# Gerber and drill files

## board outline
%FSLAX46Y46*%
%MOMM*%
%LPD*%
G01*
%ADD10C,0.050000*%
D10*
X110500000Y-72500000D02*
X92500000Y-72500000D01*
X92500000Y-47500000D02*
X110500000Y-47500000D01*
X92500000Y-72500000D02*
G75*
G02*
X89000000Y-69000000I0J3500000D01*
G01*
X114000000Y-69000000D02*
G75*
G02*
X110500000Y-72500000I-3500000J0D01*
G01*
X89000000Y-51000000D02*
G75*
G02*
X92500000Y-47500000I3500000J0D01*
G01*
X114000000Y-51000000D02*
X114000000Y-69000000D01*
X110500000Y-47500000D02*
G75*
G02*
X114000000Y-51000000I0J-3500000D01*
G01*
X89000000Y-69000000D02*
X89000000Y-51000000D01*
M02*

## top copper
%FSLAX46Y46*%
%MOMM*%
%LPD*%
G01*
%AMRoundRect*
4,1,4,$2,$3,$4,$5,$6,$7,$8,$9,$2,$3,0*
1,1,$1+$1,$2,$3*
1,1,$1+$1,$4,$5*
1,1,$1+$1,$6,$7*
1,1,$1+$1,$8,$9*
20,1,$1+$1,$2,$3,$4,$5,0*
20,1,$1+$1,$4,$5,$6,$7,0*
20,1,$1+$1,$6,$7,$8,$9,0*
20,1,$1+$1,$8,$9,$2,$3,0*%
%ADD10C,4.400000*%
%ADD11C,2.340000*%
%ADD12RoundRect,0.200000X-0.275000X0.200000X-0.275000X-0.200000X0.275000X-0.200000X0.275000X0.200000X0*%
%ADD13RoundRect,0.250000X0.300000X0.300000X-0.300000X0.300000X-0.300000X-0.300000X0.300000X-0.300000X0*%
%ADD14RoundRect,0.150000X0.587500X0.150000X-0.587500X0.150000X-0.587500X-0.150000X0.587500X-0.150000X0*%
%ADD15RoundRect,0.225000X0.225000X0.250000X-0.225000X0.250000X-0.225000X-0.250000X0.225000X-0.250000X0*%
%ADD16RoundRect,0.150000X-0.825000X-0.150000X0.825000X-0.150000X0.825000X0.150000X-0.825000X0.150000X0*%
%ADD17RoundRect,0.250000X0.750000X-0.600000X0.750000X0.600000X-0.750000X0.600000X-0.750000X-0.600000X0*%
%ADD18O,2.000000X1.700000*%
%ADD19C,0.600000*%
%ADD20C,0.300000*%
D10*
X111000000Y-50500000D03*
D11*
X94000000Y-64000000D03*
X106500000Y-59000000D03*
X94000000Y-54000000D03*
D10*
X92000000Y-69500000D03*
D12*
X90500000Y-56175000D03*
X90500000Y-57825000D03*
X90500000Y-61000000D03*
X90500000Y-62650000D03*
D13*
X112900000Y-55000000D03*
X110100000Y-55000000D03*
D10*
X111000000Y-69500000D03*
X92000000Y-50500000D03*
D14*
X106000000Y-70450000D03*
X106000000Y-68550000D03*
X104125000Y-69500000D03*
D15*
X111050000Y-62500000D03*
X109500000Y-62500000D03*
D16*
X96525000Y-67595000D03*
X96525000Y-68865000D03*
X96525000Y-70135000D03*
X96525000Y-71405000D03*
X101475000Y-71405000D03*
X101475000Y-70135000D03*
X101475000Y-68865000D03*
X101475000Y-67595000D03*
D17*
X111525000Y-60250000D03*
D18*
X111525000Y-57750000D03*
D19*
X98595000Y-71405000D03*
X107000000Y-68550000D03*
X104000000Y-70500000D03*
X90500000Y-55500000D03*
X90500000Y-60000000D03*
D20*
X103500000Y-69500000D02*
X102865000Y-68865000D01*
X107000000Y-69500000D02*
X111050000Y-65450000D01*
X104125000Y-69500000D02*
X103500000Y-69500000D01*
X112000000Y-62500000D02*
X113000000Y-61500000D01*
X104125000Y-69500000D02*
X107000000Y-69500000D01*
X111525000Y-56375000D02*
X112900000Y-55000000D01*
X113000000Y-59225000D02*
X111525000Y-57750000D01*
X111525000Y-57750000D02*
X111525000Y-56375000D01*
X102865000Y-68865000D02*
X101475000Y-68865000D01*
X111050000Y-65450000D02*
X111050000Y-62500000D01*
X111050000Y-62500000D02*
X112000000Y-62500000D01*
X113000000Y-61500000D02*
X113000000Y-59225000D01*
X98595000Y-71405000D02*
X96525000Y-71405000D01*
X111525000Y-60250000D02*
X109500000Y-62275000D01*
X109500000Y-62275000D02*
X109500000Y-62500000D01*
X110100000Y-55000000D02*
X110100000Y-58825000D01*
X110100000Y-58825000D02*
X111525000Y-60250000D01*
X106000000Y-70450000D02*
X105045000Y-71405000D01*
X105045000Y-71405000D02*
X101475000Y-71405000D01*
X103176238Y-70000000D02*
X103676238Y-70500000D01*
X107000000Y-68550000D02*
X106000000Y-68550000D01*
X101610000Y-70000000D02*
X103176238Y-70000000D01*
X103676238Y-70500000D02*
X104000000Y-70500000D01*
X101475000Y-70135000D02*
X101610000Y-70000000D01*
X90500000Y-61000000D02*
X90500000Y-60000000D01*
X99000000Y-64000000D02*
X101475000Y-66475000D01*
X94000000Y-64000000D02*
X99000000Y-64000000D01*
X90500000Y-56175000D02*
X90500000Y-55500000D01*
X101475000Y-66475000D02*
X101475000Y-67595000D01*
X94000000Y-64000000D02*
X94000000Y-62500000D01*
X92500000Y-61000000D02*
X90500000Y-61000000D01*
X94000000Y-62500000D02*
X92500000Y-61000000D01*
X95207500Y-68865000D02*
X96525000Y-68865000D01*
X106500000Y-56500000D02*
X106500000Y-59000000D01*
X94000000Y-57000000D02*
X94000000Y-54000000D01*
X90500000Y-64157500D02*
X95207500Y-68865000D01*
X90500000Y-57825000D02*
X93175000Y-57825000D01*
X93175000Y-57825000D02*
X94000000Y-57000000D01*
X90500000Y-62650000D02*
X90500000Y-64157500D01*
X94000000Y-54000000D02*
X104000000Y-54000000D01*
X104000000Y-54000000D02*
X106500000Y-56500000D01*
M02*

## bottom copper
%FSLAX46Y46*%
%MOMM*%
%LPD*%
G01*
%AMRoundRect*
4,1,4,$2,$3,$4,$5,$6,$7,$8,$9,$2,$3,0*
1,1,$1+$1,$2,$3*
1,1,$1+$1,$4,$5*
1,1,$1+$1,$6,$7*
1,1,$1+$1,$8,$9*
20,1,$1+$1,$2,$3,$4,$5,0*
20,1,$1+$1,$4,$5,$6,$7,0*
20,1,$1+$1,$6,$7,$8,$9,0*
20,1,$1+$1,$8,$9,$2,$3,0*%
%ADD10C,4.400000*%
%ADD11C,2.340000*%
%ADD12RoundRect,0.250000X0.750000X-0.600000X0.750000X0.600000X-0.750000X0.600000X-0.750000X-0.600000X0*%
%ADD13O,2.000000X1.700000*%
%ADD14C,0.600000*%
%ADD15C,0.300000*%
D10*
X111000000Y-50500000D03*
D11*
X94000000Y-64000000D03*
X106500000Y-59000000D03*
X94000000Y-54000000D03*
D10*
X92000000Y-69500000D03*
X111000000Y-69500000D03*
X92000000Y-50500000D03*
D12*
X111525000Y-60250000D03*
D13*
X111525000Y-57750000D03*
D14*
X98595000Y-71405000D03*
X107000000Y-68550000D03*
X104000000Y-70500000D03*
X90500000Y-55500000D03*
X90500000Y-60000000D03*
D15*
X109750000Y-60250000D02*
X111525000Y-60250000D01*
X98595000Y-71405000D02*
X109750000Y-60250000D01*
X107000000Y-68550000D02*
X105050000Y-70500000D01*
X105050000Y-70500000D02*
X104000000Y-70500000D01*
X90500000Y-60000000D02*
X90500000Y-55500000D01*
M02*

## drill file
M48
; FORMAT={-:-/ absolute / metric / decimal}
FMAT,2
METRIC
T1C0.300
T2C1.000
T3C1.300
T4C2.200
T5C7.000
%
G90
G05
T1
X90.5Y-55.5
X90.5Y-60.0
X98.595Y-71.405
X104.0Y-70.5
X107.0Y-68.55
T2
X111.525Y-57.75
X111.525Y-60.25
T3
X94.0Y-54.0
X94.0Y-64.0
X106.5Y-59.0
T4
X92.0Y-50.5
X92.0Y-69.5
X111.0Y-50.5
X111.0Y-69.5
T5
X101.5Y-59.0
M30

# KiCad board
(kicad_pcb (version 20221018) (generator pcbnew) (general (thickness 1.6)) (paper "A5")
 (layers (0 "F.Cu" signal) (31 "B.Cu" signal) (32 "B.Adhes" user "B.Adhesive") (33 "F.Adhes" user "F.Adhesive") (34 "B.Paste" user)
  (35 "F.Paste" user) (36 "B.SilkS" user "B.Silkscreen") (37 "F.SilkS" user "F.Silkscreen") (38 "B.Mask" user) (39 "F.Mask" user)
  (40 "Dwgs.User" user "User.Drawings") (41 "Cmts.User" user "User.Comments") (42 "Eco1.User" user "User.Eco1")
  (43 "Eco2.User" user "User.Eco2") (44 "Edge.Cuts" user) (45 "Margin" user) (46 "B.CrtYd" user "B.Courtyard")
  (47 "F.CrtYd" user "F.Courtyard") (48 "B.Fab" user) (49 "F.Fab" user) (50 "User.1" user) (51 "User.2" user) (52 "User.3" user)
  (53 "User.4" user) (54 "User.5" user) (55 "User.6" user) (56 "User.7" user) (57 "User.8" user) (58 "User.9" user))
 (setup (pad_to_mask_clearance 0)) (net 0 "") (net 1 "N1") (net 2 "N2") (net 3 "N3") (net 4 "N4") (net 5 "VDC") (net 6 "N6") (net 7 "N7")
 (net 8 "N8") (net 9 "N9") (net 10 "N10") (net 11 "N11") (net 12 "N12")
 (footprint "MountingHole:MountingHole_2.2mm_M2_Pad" (layer "F.Cu") (at 111 50.5)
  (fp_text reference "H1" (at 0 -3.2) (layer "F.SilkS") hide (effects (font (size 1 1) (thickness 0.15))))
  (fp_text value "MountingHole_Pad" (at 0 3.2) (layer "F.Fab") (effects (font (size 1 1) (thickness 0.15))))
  (pad "1" thru_hole circle (at 0 0) (size 4.4 4.4) (drill 2.2) (layers "*.Cu" "*.Mask") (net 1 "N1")))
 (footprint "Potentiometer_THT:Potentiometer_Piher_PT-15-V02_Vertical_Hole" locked (layer "F.Cu") (at 94 64)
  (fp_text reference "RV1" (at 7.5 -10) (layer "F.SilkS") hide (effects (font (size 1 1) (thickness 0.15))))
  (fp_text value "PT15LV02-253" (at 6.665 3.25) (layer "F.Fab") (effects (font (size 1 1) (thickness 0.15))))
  (pad "" np_thru_hole circle locked (at 7.5 -5) (size 7 7) (drill 7) (layers "*.Cu" "*.Mask"))
  (pad "1" thru_hole circle locked (at 0 0) (size 2.34 2.34) (drill 1.3) (layers "*.Cu" "*.Mask") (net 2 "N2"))
  (pad "2" thru_hole circle locked (at 12.5 -5) (size 2.34 2.34) (drill 1.3) (layers "*.Cu" "*.Mask") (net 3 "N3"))
  (pad "3" thru_hole circle locked (at 0 -10) (size 2.34 2.34) (drill 1.3) (layers "*.Cu" "*.Mask") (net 3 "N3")))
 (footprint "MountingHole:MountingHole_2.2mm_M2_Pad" (layer "F.Cu") (at 92 69.5)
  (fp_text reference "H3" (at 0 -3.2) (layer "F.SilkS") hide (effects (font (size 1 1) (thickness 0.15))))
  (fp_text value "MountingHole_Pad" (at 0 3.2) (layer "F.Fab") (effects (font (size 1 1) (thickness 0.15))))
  (pad "1" thru_hole circle (at 0 0) (size 4.4 4.4) (drill 2.2) (layers "*.Cu" "*.Mask") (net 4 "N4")))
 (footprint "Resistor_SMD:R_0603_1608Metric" (layer "F.Cu") (at 90.5 57 -90)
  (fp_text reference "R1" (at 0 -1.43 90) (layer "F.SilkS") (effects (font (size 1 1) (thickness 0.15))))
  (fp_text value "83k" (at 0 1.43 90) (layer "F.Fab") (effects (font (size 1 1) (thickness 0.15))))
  (pad "1" smd roundrect (at -0.825 0 270) (size 0.8 0.95) (layers "F.Cu" "F.Paste" "F.Mask") (roundrect_rratio 0.25) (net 2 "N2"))
  (pad "2" smd roundrect (at 0.825 0 270) (size 0.8 0.95) (layers "F.Cu" "F.Paste" "F.Mask") (roundrect_rratio 0.25) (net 3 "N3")))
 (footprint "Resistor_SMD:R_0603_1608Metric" (layer "F.Cu") (at 90.5 61.825 -90)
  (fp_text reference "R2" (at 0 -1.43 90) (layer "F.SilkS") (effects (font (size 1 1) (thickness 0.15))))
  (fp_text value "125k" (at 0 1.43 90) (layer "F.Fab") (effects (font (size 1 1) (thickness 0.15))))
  (pad "1" smd roundrect (at -0.825 0 270) (size 0.8 0.95) (layers "F.Cu" "F.Paste" "F.Mask") (roundrect_rratio 0.25) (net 2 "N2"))
  (pad "2" smd roundrect (at 0.825 0 270) (size 0.8 0.95) (layers "F.Cu" "F.Paste" "F.Mask") (roundrect_rratio 0.25) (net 3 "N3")))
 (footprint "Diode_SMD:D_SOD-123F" (layer "F.Cu") (at 111.5 55 180)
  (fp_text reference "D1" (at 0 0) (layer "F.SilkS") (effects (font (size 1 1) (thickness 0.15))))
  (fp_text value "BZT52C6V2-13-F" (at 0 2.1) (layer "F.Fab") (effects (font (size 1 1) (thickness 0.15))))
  (pad "1" smd roundrect (at -1.4 0 180) (size 1.1 1.1) (layers "F.Cu" "F.Paste" "F.Mask") (roundrect_rratio 0.2272727273) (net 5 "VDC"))
  (pad "2" smd roundrect (at 1.4 0 180) (size 1.1 1.1) (layers "F.Cu" "F.Paste" "F.Mask") (roundrect_rratio 0.2272727273) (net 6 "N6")))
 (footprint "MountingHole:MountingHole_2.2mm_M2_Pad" (layer "F.Cu") (at 111 69.5)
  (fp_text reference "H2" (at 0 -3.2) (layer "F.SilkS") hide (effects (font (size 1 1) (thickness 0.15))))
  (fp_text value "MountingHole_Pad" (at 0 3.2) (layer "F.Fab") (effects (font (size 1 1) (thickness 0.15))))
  (pad "1" thru_hole circle (at 0 0) (size 4.4 4.4) (drill 2.2) (layers "*.Cu" "*.Mask") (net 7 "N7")))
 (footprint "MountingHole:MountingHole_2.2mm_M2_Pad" (layer "F.Cu") (at 92 50.5)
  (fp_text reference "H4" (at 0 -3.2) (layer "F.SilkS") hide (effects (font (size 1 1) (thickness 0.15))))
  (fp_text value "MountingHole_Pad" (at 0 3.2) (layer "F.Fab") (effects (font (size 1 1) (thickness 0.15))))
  (pad "1" thru_hole circle (at 0 0) (size 4.4 4.4) (drill 2.2) (layers "*.Cu" "*.Mask") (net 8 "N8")))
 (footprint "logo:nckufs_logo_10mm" (layer "F.Cu") (at 101.5 53.5)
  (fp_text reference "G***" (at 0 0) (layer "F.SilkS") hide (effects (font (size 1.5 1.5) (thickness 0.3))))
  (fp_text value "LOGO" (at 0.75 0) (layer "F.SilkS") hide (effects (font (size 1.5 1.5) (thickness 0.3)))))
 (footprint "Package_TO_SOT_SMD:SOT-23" (layer "F.Cu") (at 105.0625 69.5 180)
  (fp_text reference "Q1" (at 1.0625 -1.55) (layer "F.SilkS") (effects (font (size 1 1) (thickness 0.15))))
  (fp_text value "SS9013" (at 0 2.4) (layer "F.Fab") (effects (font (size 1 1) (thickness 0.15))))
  (pad "1" smd roundrect (at -0.9375 -0.95 180) (size 1.475 0.6) (layers "F.Cu" "F.Paste" "F.Mask") (roundrect_rratio 0.25) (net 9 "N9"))
  (pad "2" smd roundrect (at -0.9375 0.95 180) (size 1.475 0.6) (layers "F.Cu" "F.Paste" "F.Mask") (roundrect_rratio 0.25) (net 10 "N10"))
  (pad "3" smd roundrect (at 0.9375 0 180) (size 1.475 0.6) (layers "F.Cu" "F.Paste" "F.Mask") (roundrect_rratio 0.25) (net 5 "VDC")))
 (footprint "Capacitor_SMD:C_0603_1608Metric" (layer "F.Cu") (at 110.275 62.5 180)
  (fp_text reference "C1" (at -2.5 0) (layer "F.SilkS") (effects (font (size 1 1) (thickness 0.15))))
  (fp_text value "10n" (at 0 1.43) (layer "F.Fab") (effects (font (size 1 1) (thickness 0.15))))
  (pad "1" smd roundrect (at -0.775 0 180) (size 0.9 0.95) (layers "F.Cu" "F.Paste" "F.Mask") (roundrect_rratio 0.25) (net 5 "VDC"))
  (pad "2" smd roundrect (at 0.775 0 180) (size 0.9 0.95) (layers "F.Cu" "F.Paste" "F.Mask") (roundrect_rratio 0.25) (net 6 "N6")))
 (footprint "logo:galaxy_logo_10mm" (layer "F.Cu") (at 101 64.5)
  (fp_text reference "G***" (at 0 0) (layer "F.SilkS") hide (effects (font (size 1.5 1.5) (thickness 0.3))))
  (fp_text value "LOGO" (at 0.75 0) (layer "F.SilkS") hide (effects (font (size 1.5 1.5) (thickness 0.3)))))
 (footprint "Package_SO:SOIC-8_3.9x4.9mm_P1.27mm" (layer "F.Cu") (at 99 69.5)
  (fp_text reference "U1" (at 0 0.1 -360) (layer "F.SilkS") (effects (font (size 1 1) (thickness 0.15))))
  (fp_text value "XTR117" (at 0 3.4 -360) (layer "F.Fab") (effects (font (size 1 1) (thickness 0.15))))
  (pad "1" smd roundrect (at -2.475 -1.905) (size 1.95 0.6) (layers "F.Cu" "F.Paste" "F.Mask") (roundrect_rratio 0.25) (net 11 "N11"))
  (pad "2" smd roundrect (at -2.475 -0.635) (size 1.95 0.6) (layers "F.Cu" "F.Paste" "F.Mask") (roundrect_rratio 0.25) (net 3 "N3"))
  (pad "3" smd roundrect (at -2.475 0.635) (size 1.95 0.6) (layers "F.Cu" "F.Paste" "F.Mask") (roundrect_rratio 0.25) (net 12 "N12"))
  (pad "4" smd roundrect (at -2.475 1.905) (size 1.95 0.6) (layers "F.Cu" "F.Paste" "F.Mask") (roundrect_rratio 0.25) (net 6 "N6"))
  (pad "5" smd roundrect (at 2.475 1.905) (size 1.95 0.6) (layers "F.Cu" "F.Paste" "F.Mask") (roundrect_rratio 0.25) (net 9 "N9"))
  (pad "6" smd roundrect (at 2.475 0.635) (size 1.95 0.6) (layers "F.Cu" "F.Paste" "F.Mask") (roundrect_rratio 0.25) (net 10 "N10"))
  (pad "7" smd roundrect (at 2.475 -0.635) (size 1.95 0.6) (layers "F.Cu" "F.Paste" "F.Mask") (roundrect_rratio 0.25) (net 5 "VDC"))
  (pad "8" smd roundrect (at 2.475 -1.905) (size 1.95 0.6) (layers "F.Cu" "F.Paste" "F.Mask") (roundrect_rratio 0.25) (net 2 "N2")))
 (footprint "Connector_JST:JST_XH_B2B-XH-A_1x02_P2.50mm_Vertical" (layer "B.Cu") (at 111.525 60.25 90)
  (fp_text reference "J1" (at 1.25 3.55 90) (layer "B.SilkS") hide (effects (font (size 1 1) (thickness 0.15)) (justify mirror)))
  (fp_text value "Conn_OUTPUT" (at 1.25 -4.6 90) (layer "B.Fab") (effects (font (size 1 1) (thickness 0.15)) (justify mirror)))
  (pad "1" thru_hole roundrect (at 0 0 90) (size 1.7 2) (drill 1) (layers "*.Cu" "*.Mask") (roundrect_rratio 0.147059) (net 6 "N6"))
  (pad "2" thru_hole oval (at 2.5 0 90) (size 1.7 2) (drill 1) (layers "*.Cu" "*.Mask") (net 5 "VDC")))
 (gr_line (start 110.5 72.5) (end 92.5 72.5) (stroke (width 0.05) (type default)) (layer "Edge.Cuts"))
 (gr_line (start 92.5 47.5) (end 110.5 47.5) (stroke (width 0.05) (type default)) (layer "Edge.Cuts"))
 (gr_arc (start 92.5 72.5) (mid 90.025126 71.474874) (end 89 69) (stroke (width 0.05) (type default)) (layer "Edge.Cuts"))
 (gr_arc (start 114 69) (mid 112.974874 71.474874) (end 110.5 72.5) (stroke (width 0.05) (type default)) (layer "Edge.Cuts"))
 (gr_arc (start 89 51) (mid 90.025126 48.525126) (end 92.5 47.5) (stroke (width 0.05) (type default)) (layer "Edge.Cuts"))
 (gr_line (start 114 51) (end 114 69) (stroke (width 0.05) (type default)) (layer "Edge.Cuts"))
 (gr_arc (start 110.5 47.5) (mid 112.974874 48.525126) (end 114 51) (stroke (width 0.05) (type default)) (layer "Edge.Cuts"))
 (gr_line (start 89 69) (end 89 51) (stroke (width 0.05) (type default)) (layer "Edge.Cuts"))
 (segment (start 103.5 69.5) (end 102.865 68.865) (width 0.3) (layer "F.Cu") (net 5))
 (segment (start 107 69.5) (end 111.05 65.45) (width 0.3) (layer "F.Cu") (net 5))
 (segment (start 104.125 69.5) (end 103.5 69.5) (width 0.3) (layer "F.Cu") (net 5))
 (segment (start 112 62.5) (end 113 61.5) (width 0.3) (layer "F.Cu") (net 5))
 (segment (start 104.125 69.5) (end 107 69.5) (width 0.3) (layer "F.Cu") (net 5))
 (segment (start 111.525 56.375) (end 112.9 55) (width 0.3) (layer "F.Cu") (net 5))
 (segment (start 113 59.225) (end 111.525 57.75) (width 0.3) (layer "F.Cu") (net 5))
 (segment (start 111.525 57.75) (end 111.525 56.375) (width 0.3) (layer "F.Cu") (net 5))
 (segment (start 102.865 68.865) (end 101.475 68.865) (width 0.3) (layer "F.Cu") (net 5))
 (segment (start 111.05 65.45) (end 111.05 62.5) (width 0.3) (layer "F.Cu") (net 5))
 (segment (start 111.05 62.5) (end 112 62.5) (width 0.3) (layer "F.Cu") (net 5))
 (segment (start 113 61.5) (end 113 59.225) (width 0.3) (layer "F.Cu") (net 5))
 (segment (start 98.595 71.405) (end 96.525 71.405) (width 0.3) (layer "F.Cu") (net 6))
 (segment (start 111.525 60.25) (end 109.5 62.275) (width 0.3) (layer "F.Cu") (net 6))
 (segment (start 109.5 62.275) (end 109.5 62.5) (width 0.3) (layer "F.Cu") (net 6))
 (segment (start 110.1 55) (end 110.1 58.825) (width 0.3) (layer "F.Cu") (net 6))
 (segment (start 110.1 58.825) (end 111.525 60.25) (width 0.3) (layer "F.Cu") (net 6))
 (via (at 98.595 71.405) (size 0.6) (drill 0.3) (layers "F.Cu" "B.Cu") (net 6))
 (segment (start 109.75 60.25) (end 111.525 60.25) (width 0.3) (layer "B.Cu") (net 6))
 (segment (start 98.595 71.405) (end 109.75 60.25) (width 0.3) (layer "B.Cu") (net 6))
 (segment (start 106 70.45) (end 105.045 71.405) (width 0.3) (layer "F.Cu") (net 9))
 (segment (start 105.045 71.405) (end 101.475 71.405) (width 0.3) (layer "F.Cu") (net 9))
 (segment (start 103.176238 70) (end 103.676238 70.5) (width 0.3) (layer "F.Cu") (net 10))
 (segment (start 107 68.55) (end 106 68.55) (width 0.3) (layer "F.Cu") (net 10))
 (segment (start 101.61 70) (end 103.176238 70) (width 0.3) (layer "F.Cu") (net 10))
 (segment (start 103.676238 70.5) (end 104 70.5) (width 0.3) (layer "F.Cu") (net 10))
 (segment (start 101.475 70.135) (end 101.61 70) (width 0.3) (layer "F.Cu") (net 10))
 (via (at 107 68.55) (size 0.6) (drill 0.3) (layers "F.Cu" "B.Cu") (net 10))
 (via (at 104 70.5) (size 0.6) (drill 0.3) (layers "F.Cu" "B.Cu") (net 10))
 (segment (start 107 68.55) (end 105.05 70.5) (width 0.3) (layer "B.Cu") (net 10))
 (segment (start 105.05 70.5) (end 104 70.5) (width 0.3) (layer "B.Cu") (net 10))
 (segment (start 90.5 61) (end 90.5 60) (width 0.3) (layer "F.Cu") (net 2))
 (segment (start 99 64) (end 101.475 66.475) (width 0.3) (layer "F.Cu") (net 2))
 (segment (start 94 64) (end 99 64) (width 0.3) (layer "F.Cu") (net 2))
 (segment (start 90.5 56.175) (end 90.5 55.5) (width 0.3) (layer "F.Cu") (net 2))
 (segment (start 101.475 66.475) (end 101.475 67.595) (width 0.3) (layer "F.Cu") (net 2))
 (segment (start 94 64) (end 94 62.5) (width 0.3) (layer "F.Cu") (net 2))
 (segment (start 92.5 61) (end 90.5 61) (width 0.3) (layer "F.Cu") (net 2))
 (segment (start 94 62.5) (end 92.5 61) (width 0.3) (layer "F.Cu") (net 2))
 (via (at 90.5 55.5) (size 0.6) (drill 0.3) (layers "F.Cu" "B.Cu") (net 2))
 (via (at 90.5 60) (size 0.6) (drill 0.3) (layers "F.Cu" "B.Cu") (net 2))
 (segment (start 90.5 60) (end 90.5 55.5) (width 0.3) (layer "B.Cu") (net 2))
 (segment (start 95.2075 68.865) (end 96.525 68.865) (width 0.3) (layer "F.Cu") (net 3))
 (segment (start 106.5 56.5) (end 106.5 59) (width 0.3) (layer "F.Cu") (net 3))
 (segment (start 94 57) (end 94 54) (width 0.3) (layer "F.Cu") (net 3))
 (segment (start 90.5 64.1575) (end 95.2075 68.865) (width 0.3) (layer "F.Cu") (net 3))
 (segment (start 90.5 57.825) (end 93.175 57.825) (width 0.3) (layer "F.Cu") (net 3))
 (segment (start 93.175 57.825) (end 94 57) (width 0.3) (layer "F.Cu") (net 3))
 (segment (start 90.5 62.65) (end 90.5 64.1575) (width 0.3) (layer "F.Cu") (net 3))
 (segment (start 94 54) (end 104 54) (width 0.3) (layer "F.Cu") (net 3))
 (segment (start 104 54) (end 106.5 56.5) (width 0.3) (layer "F.Cu") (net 3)))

